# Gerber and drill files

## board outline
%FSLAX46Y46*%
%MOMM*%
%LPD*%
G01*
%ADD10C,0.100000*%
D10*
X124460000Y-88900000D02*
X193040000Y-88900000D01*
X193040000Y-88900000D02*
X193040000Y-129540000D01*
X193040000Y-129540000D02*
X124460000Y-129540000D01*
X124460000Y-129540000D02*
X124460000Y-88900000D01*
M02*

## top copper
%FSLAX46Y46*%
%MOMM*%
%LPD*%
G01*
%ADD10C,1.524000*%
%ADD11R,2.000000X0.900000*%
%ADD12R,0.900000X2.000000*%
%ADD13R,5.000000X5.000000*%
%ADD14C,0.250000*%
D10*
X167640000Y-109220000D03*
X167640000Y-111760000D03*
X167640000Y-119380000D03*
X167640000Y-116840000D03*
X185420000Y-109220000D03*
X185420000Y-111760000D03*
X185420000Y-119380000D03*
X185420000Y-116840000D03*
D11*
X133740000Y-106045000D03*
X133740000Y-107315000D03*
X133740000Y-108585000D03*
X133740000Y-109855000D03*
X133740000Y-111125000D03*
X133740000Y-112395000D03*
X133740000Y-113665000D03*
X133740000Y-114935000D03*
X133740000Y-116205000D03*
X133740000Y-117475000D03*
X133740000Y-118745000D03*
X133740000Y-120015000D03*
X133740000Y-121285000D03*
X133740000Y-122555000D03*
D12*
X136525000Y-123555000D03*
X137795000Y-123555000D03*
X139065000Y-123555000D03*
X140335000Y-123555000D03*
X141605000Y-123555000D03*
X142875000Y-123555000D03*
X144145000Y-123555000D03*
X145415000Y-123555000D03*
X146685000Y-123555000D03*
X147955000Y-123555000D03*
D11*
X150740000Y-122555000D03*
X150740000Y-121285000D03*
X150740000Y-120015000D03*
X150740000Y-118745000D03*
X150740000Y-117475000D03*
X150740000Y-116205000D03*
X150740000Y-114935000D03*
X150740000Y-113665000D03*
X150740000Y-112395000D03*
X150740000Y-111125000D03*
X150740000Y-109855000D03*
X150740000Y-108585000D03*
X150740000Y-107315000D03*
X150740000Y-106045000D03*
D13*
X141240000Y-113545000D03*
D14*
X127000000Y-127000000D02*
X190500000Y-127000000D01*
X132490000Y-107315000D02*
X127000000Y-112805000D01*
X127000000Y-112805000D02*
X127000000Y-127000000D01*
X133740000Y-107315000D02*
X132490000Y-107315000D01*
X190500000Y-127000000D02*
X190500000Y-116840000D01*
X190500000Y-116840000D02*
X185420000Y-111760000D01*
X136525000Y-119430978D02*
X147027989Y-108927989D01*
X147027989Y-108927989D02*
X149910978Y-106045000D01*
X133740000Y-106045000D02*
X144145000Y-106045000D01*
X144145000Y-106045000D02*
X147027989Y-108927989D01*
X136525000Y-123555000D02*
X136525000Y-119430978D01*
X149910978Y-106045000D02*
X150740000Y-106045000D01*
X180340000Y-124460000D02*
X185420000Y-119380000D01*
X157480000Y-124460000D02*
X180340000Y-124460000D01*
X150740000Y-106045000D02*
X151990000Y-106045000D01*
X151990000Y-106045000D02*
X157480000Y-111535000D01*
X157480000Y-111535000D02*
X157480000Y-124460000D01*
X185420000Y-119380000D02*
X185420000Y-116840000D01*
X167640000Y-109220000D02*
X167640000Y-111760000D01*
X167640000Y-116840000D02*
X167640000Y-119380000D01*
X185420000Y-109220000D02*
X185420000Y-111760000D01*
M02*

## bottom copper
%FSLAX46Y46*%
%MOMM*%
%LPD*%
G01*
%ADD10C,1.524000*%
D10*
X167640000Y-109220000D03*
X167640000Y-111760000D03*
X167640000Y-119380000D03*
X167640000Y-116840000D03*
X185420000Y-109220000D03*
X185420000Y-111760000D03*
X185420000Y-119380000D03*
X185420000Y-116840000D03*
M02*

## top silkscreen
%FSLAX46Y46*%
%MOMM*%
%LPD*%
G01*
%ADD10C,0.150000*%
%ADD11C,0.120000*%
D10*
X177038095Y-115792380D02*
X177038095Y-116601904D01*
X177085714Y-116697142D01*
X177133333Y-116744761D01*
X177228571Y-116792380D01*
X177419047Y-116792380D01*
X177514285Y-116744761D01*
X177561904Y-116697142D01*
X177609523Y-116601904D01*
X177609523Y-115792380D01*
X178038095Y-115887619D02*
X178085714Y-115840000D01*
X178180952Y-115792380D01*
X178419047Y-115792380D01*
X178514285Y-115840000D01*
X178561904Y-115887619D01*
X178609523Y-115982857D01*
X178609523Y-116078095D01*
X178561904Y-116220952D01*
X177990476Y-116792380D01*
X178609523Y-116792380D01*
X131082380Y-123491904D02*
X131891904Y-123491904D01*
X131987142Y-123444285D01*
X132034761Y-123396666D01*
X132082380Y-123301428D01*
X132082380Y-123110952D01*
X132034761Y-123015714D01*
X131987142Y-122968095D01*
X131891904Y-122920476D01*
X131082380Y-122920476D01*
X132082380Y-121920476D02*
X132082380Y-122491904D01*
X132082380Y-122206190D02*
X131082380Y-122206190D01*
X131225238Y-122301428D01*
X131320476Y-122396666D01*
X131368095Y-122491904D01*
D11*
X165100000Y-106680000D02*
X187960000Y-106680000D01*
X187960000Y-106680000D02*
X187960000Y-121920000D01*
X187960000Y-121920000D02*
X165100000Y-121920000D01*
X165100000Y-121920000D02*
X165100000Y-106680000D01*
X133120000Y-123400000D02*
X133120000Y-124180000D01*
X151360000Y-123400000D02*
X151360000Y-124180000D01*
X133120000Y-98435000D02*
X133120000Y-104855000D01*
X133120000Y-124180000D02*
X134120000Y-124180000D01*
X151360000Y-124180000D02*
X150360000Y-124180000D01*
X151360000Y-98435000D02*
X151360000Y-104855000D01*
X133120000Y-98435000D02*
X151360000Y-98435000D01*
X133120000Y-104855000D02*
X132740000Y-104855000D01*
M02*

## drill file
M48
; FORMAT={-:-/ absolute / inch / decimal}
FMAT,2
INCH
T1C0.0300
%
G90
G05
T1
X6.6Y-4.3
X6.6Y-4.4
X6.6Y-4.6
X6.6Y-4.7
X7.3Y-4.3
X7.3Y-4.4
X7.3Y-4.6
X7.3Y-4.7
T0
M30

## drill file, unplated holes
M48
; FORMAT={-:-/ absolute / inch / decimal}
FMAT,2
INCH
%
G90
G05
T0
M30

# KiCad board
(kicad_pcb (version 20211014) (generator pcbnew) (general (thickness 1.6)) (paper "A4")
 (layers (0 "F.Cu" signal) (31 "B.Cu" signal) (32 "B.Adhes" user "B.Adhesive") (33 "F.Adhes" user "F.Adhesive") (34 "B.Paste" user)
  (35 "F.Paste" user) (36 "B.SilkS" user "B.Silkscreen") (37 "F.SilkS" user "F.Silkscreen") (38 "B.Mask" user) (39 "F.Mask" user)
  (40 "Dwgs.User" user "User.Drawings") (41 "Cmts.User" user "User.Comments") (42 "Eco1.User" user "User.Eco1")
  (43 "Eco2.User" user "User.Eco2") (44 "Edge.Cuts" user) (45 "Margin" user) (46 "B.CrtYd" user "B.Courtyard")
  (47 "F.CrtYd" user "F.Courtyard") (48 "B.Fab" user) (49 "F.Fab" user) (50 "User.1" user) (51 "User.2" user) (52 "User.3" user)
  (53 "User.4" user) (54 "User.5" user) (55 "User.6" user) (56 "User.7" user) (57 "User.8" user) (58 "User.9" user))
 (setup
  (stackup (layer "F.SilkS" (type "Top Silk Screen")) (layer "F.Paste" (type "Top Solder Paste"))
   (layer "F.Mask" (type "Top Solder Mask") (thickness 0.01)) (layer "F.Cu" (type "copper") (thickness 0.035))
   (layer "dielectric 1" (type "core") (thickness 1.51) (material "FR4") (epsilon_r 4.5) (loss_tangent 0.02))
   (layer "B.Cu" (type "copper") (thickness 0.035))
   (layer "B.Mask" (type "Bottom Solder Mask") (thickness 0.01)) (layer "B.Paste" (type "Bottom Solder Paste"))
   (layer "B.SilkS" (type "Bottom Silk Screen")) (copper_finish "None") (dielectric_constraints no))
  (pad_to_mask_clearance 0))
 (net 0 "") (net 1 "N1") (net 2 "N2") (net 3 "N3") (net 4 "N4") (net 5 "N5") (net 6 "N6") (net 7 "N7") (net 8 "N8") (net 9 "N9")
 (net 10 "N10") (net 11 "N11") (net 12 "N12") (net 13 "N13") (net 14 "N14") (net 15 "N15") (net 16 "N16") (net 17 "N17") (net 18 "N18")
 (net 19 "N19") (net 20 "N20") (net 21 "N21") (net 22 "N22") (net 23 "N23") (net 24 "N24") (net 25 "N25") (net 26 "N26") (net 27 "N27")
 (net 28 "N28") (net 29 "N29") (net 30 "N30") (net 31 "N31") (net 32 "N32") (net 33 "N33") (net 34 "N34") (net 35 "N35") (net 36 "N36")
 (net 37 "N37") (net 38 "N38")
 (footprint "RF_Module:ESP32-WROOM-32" (layer "F.Cu") (at 142.24 114.3)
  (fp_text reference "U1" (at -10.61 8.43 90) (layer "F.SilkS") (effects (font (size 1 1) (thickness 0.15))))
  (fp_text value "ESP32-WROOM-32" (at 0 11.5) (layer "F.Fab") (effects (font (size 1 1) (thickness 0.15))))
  (fp_line (start -9.12 9.1) (end -9.12 9.88) (layer "F.SilkS") (width 0.12))
  (fp_line (start 9.12 9.1) (end 9.12 9.88) (layer "F.SilkS") (width 0.12))
  (fp_line (start -9.12 -15.865) (end -9.12 -9.445) (layer "F.SilkS") (width 0.12))
  (fp_line (start -9.12 9.88) (end -8.12 9.88) (layer "F.SilkS") (width 0.12))
  (fp_line (start 9.12 9.88) (end 8.12 9.88) (layer "F.SilkS") (width 0.12))
  (fp_line (start 9.12 -15.865) (end 9.12 -9.445) (layer "F.SilkS") (width 0.12))
  (fp_line (start -9.12 -15.865) (end 9.12 -15.865) (layer "F.SilkS") (width 0.12))
  (fp_line (start -9.12 -9.445) (end -9.5 -9.445) (layer "F.SilkS") (width 0.12))
  (pad "1" smd rect (at -8.5 -8.255) (size 2 0.9) (layers "F.Cu" "F.Paste" "F.Mask") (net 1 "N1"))
  (pad "2" smd rect (at -8.5 -6.985) (size 2 0.9) (layers "F.Cu" "F.Paste" "F.Mask") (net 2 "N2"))
  (pad "3" smd rect (at -8.5 -5.715) (size 2 0.9) (layers "F.Cu" "F.Paste" "F.Mask") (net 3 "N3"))
  (pad "4" smd rect (at -8.5 -4.445) (size 2 0.9) (layers "F.Cu" "F.Paste" "F.Mask") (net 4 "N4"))
  (pad "5" smd rect (at -8.5 -3.175) (size 2 0.9) (layers "F.Cu" "F.Paste" "F.Mask") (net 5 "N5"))
  (pad "6" smd rect (at -8.5 -1.905) (size 2 0.9) (layers "F.Cu" "F.Paste" "F.Mask") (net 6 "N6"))
  (pad "7" smd rect (at -8.5 -0.635) (size 2 0.9) (layers "F.Cu" "F.Paste" "F.Mask") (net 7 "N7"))
  (pad "8" smd rect (at -8.5 0.635) (size 2 0.9) (layers "F.Cu" "F.Paste" "F.Mask") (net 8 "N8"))
  (pad "9" smd rect (at -8.5 1.905) (size 2 0.9) (layers "F.Cu" "F.Paste" "F.Mask") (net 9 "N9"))
  (pad "10" smd rect (at -8.5 3.175) (size 2 0.9) (layers "F.Cu" "F.Paste" "F.Mask") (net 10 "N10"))
  (pad "11" smd rect (at -8.5 4.445) (size 2 0.9) (layers "F.Cu" "F.Paste" "F.Mask") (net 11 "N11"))
  (pad "12" smd rect (at -8.5 5.715) (size 2 0.9) (layers "F.Cu" "F.Paste" "F.Mask") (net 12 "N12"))
  (pad "13" smd rect (at -8.5 6.985) (size 2 0.9) (layers "F.Cu" "F.Paste" "F.Mask") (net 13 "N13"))
  (pad "14" smd rect (at -8.5 8.255) (size 2 0.9) (layers "F.Cu" "F.Paste" "F.Mask") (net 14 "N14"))
  (pad "15" smd rect (at -5.715 9.255 90) (size 2 0.9) (layers "F.Cu" "F.Paste" "F.Mask") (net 1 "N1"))
  (pad "16" smd rect (at -4.445 9.255 90) (size 2 0.9) (layers "F.Cu" "F.Paste" "F.Mask") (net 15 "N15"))
  (pad "17" smd rect (at -3.175 9.255 90) (size 2 0.9) (layers "F.Cu" "F.Paste" "F.Mask") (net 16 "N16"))
  (pad "18" smd rect (at -1.905 9.255 90) (size 2 0.9) (layers "F.Cu" "F.Paste" "F.Mask") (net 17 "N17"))
  (pad "19" smd rect (at -0.635 9.255 90) (size 2 0.9) (layers "F.Cu" "F.Paste" "F.Mask") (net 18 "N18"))
  (pad "20" smd rect (at 0.635 9.255 90) (size 2 0.9) (layers "F.Cu" "F.Paste" "F.Mask") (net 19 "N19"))
  (pad "21" smd rect (at 1.905 9.255 90) (size 2 0.9) (layers "F.Cu" "F.Paste" "F.Mask") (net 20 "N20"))
  (pad "22" smd rect (at 3.175 9.255 90) (size 2 0.9) (layers "F.Cu" "F.Paste" "F.Mask") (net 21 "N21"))
  (pad "23" smd rect (at 4.445 9.255 90) (size 2 0.9) (layers "F.Cu" "F.Paste" "F.Mask") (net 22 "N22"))
  (pad "24" smd rect (at 5.715 9.255 90) (size 2 0.9) (layers "F.Cu" "F.Paste" "F.Mask") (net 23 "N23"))
  (pad "25" smd rect (at 8.5 8.255) (size 2 0.9) (layers "F.Cu" "F.Paste" "F.Mask") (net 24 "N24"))
  (pad "26" smd rect (at 8.5 6.985) (size 2 0.9) (layers "F.Cu" "F.Paste" "F.Mask") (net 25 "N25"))
  (pad "27" smd rect (at 8.5 5.715) (size 2 0.9) (layers "F.Cu" "F.Paste" "F.Mask") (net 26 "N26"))
  (pad "28" smd rect (at 8.5 4.445) (size 2 0.9) (layers "F.Cu" "F.Paste" "F.Mask") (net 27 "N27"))
  (pad "29" smd rect (at 8.5 3.175) (size 2 0.9) (layers "F.Cu" "F.Paste" "F.Mask") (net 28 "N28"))
  (pad "30" smd rect (at 8.5 1.905) (size 2 0.9) (layers "F.Cu" "F.Paste" "F.Mask") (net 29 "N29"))
  (pad "31" smd rect (at 8.5 0.635) (size 2 0.9) (layers "F.Cu" "F.Paste" "F.Mask") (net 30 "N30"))
  (pad "32" smd rect (at 8.5 -0.635) (size 2 0.9) (layers "F.Cu" "F.Paste" "F.Mask") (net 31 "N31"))
  (pad "33" smd rect (at 8.5 -1.905) (size 2 0.9) (layers "F.Cu" "F.Paste" "F.Mask") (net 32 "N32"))
  (pad "34" smd rect (at 8.5 -3.175) (size 2 0.9) (layers "F.Cu" "F.Paste" "F.Mask") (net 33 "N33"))
  (pad "35" smd rect (at 8.5 -4.445) (size 2 0.9) (layers "F.Cu" "F.Paste" "F.Mask") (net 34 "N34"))
  (pad "36" smd rect (at 8.5 -5.715) (size 2 0.9) (layers "F.Cu" "F.Paste" "F.Mask") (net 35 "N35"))
  (pad "37" smd rect (at 8.5 -6.985) (size 2 0.9) (layers "F.Cu" "F.Paste" "F.Mask") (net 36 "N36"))
  (pad "38" smd rect (at 8.5 -8.255) (size 2 0.9) (layers "F.Cu" "F.Paste" "F.Mask") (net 1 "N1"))
  (pad "39" smd rect (at -1 -0.755) (size 5 5) (layers "F.Cu" "F.Paste" "F.Mask") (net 1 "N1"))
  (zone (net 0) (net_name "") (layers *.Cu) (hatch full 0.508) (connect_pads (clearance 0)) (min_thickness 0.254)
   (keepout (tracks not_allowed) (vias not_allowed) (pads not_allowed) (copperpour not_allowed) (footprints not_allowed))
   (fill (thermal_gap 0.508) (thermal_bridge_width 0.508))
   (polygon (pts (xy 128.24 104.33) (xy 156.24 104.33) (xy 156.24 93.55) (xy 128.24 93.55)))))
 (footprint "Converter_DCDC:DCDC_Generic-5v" (layer "F.Cu") (at 177.8 116.84)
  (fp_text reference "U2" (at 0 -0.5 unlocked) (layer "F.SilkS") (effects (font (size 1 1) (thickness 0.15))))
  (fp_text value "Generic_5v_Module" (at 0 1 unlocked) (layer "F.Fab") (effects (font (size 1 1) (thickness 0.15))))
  (fp_line (start -12.7 5.08) (end -12.7 -10.16) (layer "F.SilkS") (width 0.12))
  (fp_line (start -12.7 -10.16) (end 10.16 -10.16) (layer "F.SilkS") (width 0.12))
  (fp_line (start 10.16 -10.16) (end 10.16 5.08) (layer "F.SilkS") (width 0.12))
  (fp_line (start 10.16 5.08) (end -12.7 5.08) (layer "F.SilkS") (width 0.12))
  (pad "1" thru_hole circle (at -10.16 -5.08) (size 1.524 1.524) (drill 0.762) (layers *.Cu *.Mask) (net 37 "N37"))
  (pad "1" thru_hole circle (at -10.16 -7.62) (size 1.524 1.524) (drill 0.762) (layers *.Cu *.Mask) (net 37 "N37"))
  (pad "2" thru_hole circle (at -10.16 2.54) (size 1.524 1.524) (drill 0.762) (layers *.Cu *.Mask) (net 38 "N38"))
  (pad "2" thru_hole circle (at -10.16 0) (size 1.524 1.524) (drill 0.762) (layers *.Cu *.Mask) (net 38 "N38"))
  (pad "3" thru_hole circle (at 7.62 -7.62) (size 1.524 1.524) (drill 0.762) (layers *.Cu *.Mask) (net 2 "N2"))
  (pad "3" thru_hole circle (at 7.62 -5.08) (size 1.524 1.524) (drill 0.762) (layers *.Cu *.Mask) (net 2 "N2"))
  (pad "4" thru_hole circle (at 7.62 2.54) (size 1.524 1.524) (drill 0.762) (layers *.Cu *.Mask) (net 1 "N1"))
  (pad "4" thru_hole circle (at 7.62 0) (size 1.524 1.524) (drill 0.762) (layers *.Cu *.Mask) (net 1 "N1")))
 (gr_rect (start 124.46 88.9) (end 193.04 129.54) (layer "Edge.Cuts") (width 0.1) (fill none))
 (segment (start 144.145 106.045) (end 147.027989 108.927989) (width 0.25) (layer "F.Cu") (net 1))
 (segment (start 157.48 124.46) (end 180.34 124.46) (width 0.25) (layer "F.Cu") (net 1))
 (segment (start 147.027989 108.927989) (end 149.910978 106.045) (width 0.25) (layer "F.Cu") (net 1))
 (segment (start 149.910978 106.045) (end 150.74 106.045) (width 0.25) (layer "F.Cu") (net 1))
 (segment (start 150.74 106.045) (end 151.99 106.045) (width 0.25) (layer "F.Cu") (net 1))
 (segment (start 157.48 111.535) (end 157.48 124.46) (width 0.25) (layer "F.Cu") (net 1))
 (segment (start 180.34 124.46) (end 185.42 119.38) (width 0.25) (layer "F.Cu") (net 1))
 (segment (start 133.74 106.045) (end 144.145 106.045) (width 0.25) (layer "F.Cu") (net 1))
 (segment (start 185.42 119.38) (end 185.42 116.84) (width 0.25) (layer "F.Cu") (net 1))
 (segment (start 151.99 106.045) (end 157.48 111.535) (width 0.25) (layer "F.Cu") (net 1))
 (segment (start 136.525 119.430978) (end 147.027989 108.927989) (width 0.25) (layer "F.Cu") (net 1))
 (segment (start 136.525 123.555) (end 136.525 119.430978) (width 0.25) (layer "F.Cu") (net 1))
 (segment (start 185.42 109.22) (end 185.42 111.76) (width 0.25) (layer "F.Cu") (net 2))
 (segment (start 133.74 107.315) (end 132.49 107.315) (width 0.25) (layer "F.Cu") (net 2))
 (segment (start 190.5 127) (end 190.5 116.84) (width 0.25) (layer "F.Cu") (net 2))
 (segment (start 132.49 107.315) (end 127 112.805) (width 0.25) (layer "F.Cu") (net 2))
 (segment (start 127 112.805) (end 127 127) (width 0.25) (layer "F.Cu") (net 2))
 (segment (start 190.5 116.84) (end 185.42 111.76) (width 0.25) (layer "F.Cu") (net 2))
 (segment (start 127 127) (end 190.5 127) (width 0.25) (layer "F.Cu") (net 2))
 (segment (start 167.64 109.22) (end 167.64 111.76) (width 0.25) (layer "F.Cu") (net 37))
 (segment (start 167.64 116.84) (end 167.64 119.38) (width 0.25) (layer "F.Cu") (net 38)))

